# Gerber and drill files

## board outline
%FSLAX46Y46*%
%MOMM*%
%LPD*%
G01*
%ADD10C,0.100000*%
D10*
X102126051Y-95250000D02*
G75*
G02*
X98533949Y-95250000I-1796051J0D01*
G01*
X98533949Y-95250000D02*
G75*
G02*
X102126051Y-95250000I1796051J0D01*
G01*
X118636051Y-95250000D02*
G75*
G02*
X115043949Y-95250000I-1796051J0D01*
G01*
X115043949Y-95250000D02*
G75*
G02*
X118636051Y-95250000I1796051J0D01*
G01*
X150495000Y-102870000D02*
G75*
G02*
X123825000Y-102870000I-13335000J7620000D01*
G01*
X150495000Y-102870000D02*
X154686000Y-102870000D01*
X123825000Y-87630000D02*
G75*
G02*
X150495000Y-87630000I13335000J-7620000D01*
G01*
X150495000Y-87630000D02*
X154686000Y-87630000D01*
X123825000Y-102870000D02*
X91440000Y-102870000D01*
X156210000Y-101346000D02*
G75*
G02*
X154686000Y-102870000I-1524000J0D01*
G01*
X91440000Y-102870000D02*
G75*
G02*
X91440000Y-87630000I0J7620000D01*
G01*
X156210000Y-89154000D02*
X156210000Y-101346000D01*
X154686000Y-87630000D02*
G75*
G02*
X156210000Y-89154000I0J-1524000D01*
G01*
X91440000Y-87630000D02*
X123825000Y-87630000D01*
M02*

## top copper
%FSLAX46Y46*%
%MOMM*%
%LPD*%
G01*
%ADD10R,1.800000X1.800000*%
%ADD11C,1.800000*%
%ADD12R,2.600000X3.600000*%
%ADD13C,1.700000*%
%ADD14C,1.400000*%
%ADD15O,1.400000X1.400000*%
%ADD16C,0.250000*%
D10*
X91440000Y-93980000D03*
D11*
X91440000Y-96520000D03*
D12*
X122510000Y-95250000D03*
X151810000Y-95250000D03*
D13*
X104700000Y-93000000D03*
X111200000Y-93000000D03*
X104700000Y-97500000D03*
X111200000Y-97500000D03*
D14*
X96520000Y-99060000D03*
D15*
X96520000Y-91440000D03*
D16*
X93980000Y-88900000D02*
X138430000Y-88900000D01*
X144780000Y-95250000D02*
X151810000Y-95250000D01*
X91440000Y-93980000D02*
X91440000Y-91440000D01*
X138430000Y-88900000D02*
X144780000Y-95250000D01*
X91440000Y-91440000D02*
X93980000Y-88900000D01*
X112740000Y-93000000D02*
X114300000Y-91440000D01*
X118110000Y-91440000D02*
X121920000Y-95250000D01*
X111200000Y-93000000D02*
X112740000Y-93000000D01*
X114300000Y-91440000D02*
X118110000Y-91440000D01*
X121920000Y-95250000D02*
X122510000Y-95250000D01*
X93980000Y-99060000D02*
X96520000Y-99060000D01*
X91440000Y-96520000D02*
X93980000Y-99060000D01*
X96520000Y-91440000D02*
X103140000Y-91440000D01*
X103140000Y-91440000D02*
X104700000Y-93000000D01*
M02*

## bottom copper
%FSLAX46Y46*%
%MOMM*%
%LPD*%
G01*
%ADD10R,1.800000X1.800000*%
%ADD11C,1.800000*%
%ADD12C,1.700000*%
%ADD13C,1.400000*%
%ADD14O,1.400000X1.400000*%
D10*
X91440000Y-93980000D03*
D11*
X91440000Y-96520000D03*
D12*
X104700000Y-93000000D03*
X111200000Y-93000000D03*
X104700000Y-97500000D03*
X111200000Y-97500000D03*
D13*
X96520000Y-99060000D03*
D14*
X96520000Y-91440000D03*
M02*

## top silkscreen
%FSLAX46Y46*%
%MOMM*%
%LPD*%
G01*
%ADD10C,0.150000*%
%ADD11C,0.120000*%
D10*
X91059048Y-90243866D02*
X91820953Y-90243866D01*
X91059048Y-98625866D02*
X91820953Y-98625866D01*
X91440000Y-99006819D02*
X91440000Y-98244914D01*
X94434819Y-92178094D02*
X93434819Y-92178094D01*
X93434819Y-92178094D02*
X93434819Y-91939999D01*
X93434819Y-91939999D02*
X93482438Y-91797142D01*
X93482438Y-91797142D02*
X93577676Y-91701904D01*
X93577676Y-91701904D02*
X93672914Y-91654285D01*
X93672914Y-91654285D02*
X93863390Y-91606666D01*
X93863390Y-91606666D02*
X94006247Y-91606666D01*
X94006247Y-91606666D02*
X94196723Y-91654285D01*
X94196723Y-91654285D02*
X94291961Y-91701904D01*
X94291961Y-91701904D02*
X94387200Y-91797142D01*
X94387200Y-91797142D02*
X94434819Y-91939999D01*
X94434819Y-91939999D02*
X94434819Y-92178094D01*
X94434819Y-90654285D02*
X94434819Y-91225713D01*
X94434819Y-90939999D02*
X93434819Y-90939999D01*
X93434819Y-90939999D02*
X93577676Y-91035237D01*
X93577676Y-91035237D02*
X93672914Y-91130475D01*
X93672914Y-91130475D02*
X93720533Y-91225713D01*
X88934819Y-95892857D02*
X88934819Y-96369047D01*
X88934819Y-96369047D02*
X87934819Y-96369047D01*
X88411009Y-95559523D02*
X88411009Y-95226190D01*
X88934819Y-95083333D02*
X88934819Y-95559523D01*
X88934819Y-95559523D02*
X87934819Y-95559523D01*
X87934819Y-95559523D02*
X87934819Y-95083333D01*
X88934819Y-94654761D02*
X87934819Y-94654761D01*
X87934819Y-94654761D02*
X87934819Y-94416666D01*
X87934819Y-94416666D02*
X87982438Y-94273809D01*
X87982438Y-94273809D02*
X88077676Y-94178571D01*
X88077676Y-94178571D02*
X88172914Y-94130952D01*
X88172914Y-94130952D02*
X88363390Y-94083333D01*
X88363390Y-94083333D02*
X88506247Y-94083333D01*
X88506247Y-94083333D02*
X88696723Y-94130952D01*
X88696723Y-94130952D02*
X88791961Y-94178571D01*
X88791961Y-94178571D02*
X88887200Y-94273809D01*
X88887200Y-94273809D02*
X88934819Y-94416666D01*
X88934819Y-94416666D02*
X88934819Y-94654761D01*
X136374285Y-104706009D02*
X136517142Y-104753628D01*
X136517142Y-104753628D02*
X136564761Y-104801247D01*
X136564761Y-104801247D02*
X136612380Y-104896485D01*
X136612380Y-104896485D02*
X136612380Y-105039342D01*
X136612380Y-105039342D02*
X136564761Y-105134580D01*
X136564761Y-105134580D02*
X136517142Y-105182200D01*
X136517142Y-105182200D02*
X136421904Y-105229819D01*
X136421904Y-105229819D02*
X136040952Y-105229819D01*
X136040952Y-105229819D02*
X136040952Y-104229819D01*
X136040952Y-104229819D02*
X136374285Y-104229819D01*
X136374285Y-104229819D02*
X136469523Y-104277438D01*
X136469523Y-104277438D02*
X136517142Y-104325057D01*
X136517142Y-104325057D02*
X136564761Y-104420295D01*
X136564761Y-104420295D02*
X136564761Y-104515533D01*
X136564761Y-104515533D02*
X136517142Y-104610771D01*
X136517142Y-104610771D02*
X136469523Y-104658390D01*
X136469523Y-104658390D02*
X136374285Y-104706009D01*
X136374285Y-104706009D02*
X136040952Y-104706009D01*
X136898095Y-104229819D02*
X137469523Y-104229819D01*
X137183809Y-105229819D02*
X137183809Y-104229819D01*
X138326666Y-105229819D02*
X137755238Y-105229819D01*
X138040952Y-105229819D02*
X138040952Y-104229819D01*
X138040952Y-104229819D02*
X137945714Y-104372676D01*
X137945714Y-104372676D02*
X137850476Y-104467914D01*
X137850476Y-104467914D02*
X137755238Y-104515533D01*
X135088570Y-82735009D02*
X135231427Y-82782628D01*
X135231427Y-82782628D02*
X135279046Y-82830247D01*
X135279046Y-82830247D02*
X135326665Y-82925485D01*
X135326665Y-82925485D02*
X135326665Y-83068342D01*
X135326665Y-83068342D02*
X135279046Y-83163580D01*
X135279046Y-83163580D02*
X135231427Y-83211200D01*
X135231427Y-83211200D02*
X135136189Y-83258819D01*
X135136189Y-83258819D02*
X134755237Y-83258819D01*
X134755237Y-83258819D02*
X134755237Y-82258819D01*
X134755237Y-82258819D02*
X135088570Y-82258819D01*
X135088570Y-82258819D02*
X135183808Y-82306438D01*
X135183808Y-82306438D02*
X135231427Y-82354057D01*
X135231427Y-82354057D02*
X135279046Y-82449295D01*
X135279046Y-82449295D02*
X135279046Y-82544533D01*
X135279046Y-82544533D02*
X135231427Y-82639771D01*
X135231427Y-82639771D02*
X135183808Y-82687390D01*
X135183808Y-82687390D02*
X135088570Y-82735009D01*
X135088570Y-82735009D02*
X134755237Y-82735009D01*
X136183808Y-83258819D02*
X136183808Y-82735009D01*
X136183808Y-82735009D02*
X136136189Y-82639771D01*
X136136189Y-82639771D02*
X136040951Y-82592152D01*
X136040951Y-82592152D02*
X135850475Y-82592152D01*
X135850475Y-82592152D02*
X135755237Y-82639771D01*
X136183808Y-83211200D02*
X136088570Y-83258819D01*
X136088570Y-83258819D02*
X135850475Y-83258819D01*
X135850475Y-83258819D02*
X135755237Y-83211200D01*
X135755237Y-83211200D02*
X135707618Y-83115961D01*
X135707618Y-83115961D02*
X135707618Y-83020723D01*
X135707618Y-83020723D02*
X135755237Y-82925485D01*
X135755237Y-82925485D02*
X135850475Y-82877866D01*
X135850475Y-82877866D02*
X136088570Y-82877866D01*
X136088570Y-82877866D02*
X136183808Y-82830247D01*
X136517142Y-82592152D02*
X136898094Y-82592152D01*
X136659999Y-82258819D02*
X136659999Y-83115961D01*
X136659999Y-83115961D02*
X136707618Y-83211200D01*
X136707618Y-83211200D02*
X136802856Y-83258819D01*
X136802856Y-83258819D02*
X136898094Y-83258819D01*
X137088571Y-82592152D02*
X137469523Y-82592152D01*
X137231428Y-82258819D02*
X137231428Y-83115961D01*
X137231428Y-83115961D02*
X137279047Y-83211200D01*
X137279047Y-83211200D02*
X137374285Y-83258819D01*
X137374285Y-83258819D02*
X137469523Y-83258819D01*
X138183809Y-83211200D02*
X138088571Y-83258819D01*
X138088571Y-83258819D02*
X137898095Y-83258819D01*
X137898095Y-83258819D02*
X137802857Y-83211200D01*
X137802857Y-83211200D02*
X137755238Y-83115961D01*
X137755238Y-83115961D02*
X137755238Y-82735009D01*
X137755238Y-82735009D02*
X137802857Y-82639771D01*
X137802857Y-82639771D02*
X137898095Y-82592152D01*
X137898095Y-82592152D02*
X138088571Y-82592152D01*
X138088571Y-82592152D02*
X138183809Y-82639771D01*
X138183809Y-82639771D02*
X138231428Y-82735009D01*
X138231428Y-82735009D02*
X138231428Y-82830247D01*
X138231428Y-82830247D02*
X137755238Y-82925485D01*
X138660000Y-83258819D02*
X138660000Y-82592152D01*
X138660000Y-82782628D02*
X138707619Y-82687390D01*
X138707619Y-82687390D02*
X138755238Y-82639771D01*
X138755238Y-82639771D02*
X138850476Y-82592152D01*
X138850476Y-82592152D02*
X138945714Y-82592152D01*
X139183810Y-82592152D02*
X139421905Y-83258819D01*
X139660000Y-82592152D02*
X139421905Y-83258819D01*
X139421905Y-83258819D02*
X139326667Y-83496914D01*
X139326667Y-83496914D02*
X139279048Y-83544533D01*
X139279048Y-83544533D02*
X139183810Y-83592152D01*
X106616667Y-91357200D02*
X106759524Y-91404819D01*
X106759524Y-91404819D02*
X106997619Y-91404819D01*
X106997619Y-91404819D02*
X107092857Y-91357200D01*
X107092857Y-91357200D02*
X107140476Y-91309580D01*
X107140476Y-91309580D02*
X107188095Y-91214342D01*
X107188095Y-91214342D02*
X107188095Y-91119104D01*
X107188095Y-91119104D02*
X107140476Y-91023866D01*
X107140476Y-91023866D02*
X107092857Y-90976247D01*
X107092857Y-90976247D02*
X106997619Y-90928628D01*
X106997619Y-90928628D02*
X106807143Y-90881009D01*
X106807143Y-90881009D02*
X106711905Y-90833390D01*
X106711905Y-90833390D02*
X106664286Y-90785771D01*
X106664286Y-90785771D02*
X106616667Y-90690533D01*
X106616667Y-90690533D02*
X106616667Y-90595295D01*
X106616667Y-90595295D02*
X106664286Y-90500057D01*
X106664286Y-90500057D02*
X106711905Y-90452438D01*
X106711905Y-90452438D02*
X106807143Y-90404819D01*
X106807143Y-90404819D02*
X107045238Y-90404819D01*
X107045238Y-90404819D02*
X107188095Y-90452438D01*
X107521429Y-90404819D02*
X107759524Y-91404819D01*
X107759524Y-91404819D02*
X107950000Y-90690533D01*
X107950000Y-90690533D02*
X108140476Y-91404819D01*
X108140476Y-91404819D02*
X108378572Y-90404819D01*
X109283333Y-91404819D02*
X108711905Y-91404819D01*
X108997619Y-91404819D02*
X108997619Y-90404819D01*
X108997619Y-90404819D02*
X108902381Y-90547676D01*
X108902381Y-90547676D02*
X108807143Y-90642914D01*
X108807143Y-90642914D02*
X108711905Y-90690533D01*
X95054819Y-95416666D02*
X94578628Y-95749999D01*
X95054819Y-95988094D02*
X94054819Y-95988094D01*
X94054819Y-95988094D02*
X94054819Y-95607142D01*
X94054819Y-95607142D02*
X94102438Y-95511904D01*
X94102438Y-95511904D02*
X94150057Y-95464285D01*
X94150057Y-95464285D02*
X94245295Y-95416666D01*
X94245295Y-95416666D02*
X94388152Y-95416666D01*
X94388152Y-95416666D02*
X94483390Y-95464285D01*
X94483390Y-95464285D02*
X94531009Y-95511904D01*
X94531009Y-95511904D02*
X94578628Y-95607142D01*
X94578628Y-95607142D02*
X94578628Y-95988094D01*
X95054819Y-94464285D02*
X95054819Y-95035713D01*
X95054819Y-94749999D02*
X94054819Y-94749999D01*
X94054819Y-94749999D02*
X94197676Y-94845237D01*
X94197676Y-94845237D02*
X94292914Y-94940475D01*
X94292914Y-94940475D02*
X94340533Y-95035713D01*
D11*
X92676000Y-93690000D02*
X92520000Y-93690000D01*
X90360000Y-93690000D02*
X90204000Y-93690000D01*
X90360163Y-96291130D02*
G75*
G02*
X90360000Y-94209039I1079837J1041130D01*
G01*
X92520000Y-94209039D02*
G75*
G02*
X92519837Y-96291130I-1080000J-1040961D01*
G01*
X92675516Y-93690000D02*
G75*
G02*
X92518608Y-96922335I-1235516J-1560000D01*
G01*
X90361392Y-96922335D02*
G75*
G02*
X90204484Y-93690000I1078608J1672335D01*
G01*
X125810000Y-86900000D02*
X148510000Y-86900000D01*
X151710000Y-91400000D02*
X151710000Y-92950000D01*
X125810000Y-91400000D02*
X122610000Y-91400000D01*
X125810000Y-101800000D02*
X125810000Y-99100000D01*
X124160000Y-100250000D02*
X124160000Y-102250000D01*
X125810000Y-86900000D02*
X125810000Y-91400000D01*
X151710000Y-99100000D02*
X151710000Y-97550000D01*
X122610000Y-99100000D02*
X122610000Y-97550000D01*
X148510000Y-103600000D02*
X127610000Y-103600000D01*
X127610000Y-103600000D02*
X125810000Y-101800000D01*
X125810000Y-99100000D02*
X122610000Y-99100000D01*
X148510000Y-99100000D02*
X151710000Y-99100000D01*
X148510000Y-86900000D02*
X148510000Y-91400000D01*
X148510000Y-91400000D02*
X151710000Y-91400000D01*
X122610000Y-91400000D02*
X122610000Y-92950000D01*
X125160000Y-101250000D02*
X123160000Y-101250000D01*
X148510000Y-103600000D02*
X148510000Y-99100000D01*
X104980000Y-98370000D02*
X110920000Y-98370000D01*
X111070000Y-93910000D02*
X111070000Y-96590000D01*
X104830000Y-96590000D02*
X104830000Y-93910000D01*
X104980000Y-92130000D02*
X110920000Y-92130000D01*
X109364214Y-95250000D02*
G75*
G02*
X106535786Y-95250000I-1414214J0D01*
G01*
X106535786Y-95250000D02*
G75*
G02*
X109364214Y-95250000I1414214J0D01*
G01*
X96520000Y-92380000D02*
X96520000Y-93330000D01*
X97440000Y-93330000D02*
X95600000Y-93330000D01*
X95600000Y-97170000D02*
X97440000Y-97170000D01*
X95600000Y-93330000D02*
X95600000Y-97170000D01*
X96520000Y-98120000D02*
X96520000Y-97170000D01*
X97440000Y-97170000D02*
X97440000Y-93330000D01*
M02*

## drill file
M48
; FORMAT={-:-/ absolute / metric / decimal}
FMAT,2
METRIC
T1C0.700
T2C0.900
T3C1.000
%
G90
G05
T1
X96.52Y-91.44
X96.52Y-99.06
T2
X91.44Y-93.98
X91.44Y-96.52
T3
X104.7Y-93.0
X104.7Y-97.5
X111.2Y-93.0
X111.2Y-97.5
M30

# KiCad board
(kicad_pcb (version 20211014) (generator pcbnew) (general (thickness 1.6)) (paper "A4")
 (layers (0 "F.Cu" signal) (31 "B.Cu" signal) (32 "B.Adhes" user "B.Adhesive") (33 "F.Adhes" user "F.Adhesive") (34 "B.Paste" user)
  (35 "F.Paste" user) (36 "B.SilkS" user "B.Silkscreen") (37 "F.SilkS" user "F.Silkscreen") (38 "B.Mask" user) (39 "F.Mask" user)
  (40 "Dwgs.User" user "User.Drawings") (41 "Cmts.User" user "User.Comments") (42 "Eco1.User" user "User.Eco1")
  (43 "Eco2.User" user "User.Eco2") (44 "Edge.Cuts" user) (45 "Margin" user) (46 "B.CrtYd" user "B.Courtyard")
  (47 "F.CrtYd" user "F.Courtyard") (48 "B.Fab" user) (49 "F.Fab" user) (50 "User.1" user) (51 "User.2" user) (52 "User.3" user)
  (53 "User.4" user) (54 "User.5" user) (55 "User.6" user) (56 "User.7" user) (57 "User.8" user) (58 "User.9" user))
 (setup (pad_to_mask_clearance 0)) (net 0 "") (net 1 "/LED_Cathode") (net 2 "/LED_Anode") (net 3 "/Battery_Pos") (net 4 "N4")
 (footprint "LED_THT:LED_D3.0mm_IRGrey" (layer "F.Cu") (at 91.44 93.98 -90)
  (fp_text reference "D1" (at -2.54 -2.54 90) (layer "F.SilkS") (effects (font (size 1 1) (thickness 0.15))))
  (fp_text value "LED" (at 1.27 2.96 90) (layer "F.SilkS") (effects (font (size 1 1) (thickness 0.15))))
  (fp_line (start -0.29 -1.236) (end -0.29 -1.08) (layer "F.SilkS") (width 0.12))
  (fp_line (start -0.29 1.08) (end -0.29 1.236) (layer "F.SilkS") (width 0.12))
  (fp_arc (start 2.31113 1.079837) (mid 1.270117 1.5) (end 0.229039 1.08) (layer "F.SilkS") (width 0.12))
  (fp_arc (start 0.229039 -1.08) (mid 1.270117 -1.5) (end 2.31113 -1.079837) (layer "F.SilkS") (width 0.12))
  (fp_arc (start -0.29 -1.235516) (mid 1.366487 -1.987659) (end 2.942335 -1.078608) (layer "F.SilkS") (width 0.12))
  (fp_arc (start 2.942335 1.078608) (mid 1.366487 1.987659) (end -0.29 1.235516) (layer "F.SilkS") (width 0.12))
  (pad "1" thru_hole rect locked (at 0 0 270) (size 1.8 1.8) (drill 0.9) (layers *.Cu *.Mask) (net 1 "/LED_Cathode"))
  (pad "2" thru_hole circle locked (at 2.54 0 270) (size 1.8 1.8) (drill 0.9) (layers *.Cu *.Mask) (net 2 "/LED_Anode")))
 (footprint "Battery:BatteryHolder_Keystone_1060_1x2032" (layer "F.Cu") (at 137.16 95.25)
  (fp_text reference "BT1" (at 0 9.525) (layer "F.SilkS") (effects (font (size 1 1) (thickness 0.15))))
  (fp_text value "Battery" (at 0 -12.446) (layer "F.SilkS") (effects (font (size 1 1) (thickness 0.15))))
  (fp_line (start -11.35 -8.35) (end 11.35 -8.35) (layer "F.SilkS") (width 0.12))
  (fp_line (start 14.55 -3.85) (end 14.55 -2.3) (layer "F.SilkS") (width 0.12))
  (fp_line (start -11.35 -3.85) (end -14.55 -3.85) (layer "F.SilkS") (width 0.12))
  (fp_line (start -11.35 6.55) (end -11.35 3.85) (layer "F.SilkS") (width 0.12))
  (fp_line (start -13 5) (end -13 7) (layer "F.SilkS") (width 0.12))
  (fp_line (start -11.35 -8.35) (end -11.35 -3.85) (layer "F.SilkS") (width 0.12))
  (fp_line (start 14.55 3.85) (end 14.55 2.3) (layer "F.SilkS") (width 0.12))
  (fp_line (start -14.55 3.85) (end -14.55 2.3) (layer "F.SilkS") (width 0.12))
  (fp_line (start 11.35 8.35) (end -9.55 8.35) (layer "F.SilkS") (width 0.12))
  (fp_line (start -9.55 8.35) (end -11.35 6.55) (layer "F.SilkS") (width 0.12))
  (fp_line (start -11.35 3.85) (end -14.55 3.85) (layer "F.SilkS") (width 0.12))
  (fp_line (start 11.35 3.85) (end 14.55 3.85) (layer "F.SilkS") (width 0.12))
  (fp_line (start 11.35 -8.35) (end 11.35 -3.85) (layer "F.SilkS") (width 0.12))
  (fp_line (start 11.35 -3.85) (end 14.55 -3.85) (layer "F.SilkS") (width 0.12))
  (fp_line (start -14.55 -3.85) (end -14.55 -2.3) (layer "F.SilkS") (width 0.12))
  (fp_line (start -12 6) (end -14 6) (layer "F.SilkS") (width 0.12))
  (fp_line (start 11.35 8.35) (end 11.35 3.85) (layer "F.SilkS") (width 0.12))
  (pad "1" smd rect locked (at -14.65 0 180) (size 2.6 3.6) (layers "F.Cu" "F.Paste" "F.Mask") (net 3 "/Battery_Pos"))
  (pad "2" smd rect locked (at 14.65 0 180) (size 2.6 3.6) (layers "F.Cu" "F.Paste" "F.Mask") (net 1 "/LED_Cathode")))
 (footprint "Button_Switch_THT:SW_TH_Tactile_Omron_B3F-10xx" (layer "F.Cu") (at 104.7 93)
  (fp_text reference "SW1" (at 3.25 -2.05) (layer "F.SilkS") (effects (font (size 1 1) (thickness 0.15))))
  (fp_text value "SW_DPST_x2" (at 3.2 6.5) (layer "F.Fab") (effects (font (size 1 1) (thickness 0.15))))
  (fp_line (start 0.28 5.37) (end 6.22 5.37) (layer "F.SilkS") (width 0.12))
  (fp_line (start 6.37 0.91) (end 6.37 3.59) (layer "F.SilkS") (width 0.12))
  (fp_line (start 0.13 3.59) (end 0.13 0.91) (layer "F.SilkS") (width 0.12))
  (fp_line (start 0.28 -0.87) (end 6.22 -0.87) (layer "F.SilkS") (width 0.12))
  (fp_circle (center 3.25 2.25) (end 4.25 3.25) (layer "F.SilkS") (width 0.12) (fill none))
  (pad "1" thru_hole circle locked (at 0 0) (size 1.7 1.7) (drill 1) (layers *.Cu *.Mask) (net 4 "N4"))
  (pad "2" thru_hole circle locked (at 6.5 0) (size 1.7 1.7) (drill 1) (layers *.Cu *.Mask) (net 3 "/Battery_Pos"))
  (pad "3" thru_hole circle locked (at 0 4.5) (size 1.7 1.7) (drill 1) (layers *.Cu *.Mask))
  (pad "4" thru_hole circle locked (at 6.5 4.5) (size 1.7 1.7) (drill 1) (layers *.Cu *.Mask)))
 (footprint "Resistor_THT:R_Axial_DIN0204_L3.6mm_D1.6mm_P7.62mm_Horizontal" (layer "F.Cu") (at 96.52 99.06 90)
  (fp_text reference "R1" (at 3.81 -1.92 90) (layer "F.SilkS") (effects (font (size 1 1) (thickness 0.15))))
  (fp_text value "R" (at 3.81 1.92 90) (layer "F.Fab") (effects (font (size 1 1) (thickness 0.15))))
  (fp_line (start 6.68 0) (end 5.73 0) (layer "F.SilkS") (width 0.12))
  (fp_line (start 5.73 0.92) (end 5.73 -0.92) (layer "F.SilkS") (width 0.12))
  (fp_line (start 1.89 -0.92) (end 1.89 0.92) (layer "F.SilkS") (width 0.12))
  (fp_line (start 5.73 -0.92) (end 1.89 -0.92) (layer "F.SilkS") (width 0.12))
  (fp_line (start 0.94 0) (end 1.89 0) (layer "F.SilkS") (width 0.12))
  (fp_line (start 1.89 0.92) (end 5.73 0.92) (layer "F.SilkS") (width 0.12))
  (pad "1" thru_hole circle locked (at 0 0 90) (size 1.4 1.4) (drill 0.7) (layers *.Cu *.Mask) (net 2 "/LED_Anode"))
  (pad "2" thru_hole oval locked (at 7.62 0 90) (size 1.4 1.4) (drill 0.7) (layers *.Cu *.Mask) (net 4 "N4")))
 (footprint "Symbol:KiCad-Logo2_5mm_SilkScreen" (layer "B.Cu") (at 136.398 93.98 180)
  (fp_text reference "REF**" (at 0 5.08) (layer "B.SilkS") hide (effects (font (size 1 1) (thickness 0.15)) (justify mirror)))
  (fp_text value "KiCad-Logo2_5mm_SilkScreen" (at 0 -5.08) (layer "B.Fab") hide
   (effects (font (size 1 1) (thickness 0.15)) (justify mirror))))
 (gr_circle (center 100.33 95.25) (end 101.6 96.52) (layer "Edge.Cuts") (width 0.1) (fill none))
 (gr_circle (center 116.84 95.25) (end 118.11 93.98) (layer "Edge.Cuts") (width 0.1) (fill none))
 (gr_arc (start 150.495 102.87) (mid 137.16 110.608601) (end 123.825 102.87) (layer "Edge.Cuts") (width 0.1))
 (gr_line (start 150.495 102.87) (end 154.686 102.87) (layer "Edge.Cuts") (width 0.1))
 (gr_arc (start 123.825 87.63) (mid 137.16 79.891399) (end 150.495 87.63) (layer "Edge.Cuts") (width 0.1))
 (gr_line (start 150.495 87.63) (end 154.686 87.63) (layer "Edge.Cuts") (width 0.1))
 (gr_line (start 123.825 102.87) (end 91.44 102.87) (layer "Edge.Cuts") (width 0.1))
 (gr_arc (start 156.21 101.346) (mid 155.763631 102.423631) (end 154.686 102.87) (layer "Edge.Cuts") (width 0.1))
 (gr_arc (start 91.44 102.87) (mid 83.82 95.25) (end 91.44 87.63) (layer "Edge.Cuts") (width 0.1))
 (gr_line (start 156.21 89.154) (end 156.21 101.346) (layer "Edge.Cuts") (width 0.1))
 (gr_arc (start 154.686 87.63) (mid 155.763631 88.076369) (end 156.21 89.154) (layer "Edge.Cuts") (width 0.1))
 (gr_line (start 91.44 87.63) (end 123.825 87.63) (layer "Edge.Cuts") (width 0.1))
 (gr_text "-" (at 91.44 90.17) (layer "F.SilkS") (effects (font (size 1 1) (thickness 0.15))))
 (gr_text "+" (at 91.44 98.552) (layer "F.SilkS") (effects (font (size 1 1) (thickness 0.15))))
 (segment (start 93.98 88.9) (end 138.43 88.9) (width 0.25) (layer "F.Cu") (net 1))
 (segment (start 144.78 95.25) (end 151.81 95.25) (width 0.25) (layer "F.Cu") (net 1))
 (segment (start 91.44 93.98) (end 91.44 91.44) (width 0.25) (layer "F.Cu") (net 1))
 (segment (start 138.43 88.9) (end 144.78 95.25) (width 0.25) (layer "F.Cu") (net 1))
 (segment (start 91.44 91.44) (end 93.98 88.9) (width 0.25) (layer "F.Cu") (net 1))
 (segment (start 112.74 93) (end 114.3 91.44) (width 0.25) (layer "F.Cu") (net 3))
 (segment (start 118.11 91.44) (end 121.92 95.25) (width 0.25) (layer "F.Cu") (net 3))
 (segment (start 111.2 93) (end 112.74 93) (width 0.25) (layer "F.Cu") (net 3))
 (segment (start 114.3 91.44) (end 118.11 91.44) (width 0.25) (layer "F.Cu") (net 3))
 (segment (start 121.92 95.25) (end 122.51 95.25) (width 0.25) (layer "F.Cu") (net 3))
 (segment (start 93.98 99.06) (end 96.52 99.06) (width 0.25) (layer "F.Cu") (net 2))
 (segment (start 91.44 96.52) (end 93.98 99.06) (width 0.25) (layer "F.Cu") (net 2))
 (segment (start 96.52 91.44) (end 103.14 91.44) (width 0.25) (layer "F.Cu") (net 4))
 (segment (start 103.14 91.44) (end 104.7 93) (width 0.25) (layer "F.Cu") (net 4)))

